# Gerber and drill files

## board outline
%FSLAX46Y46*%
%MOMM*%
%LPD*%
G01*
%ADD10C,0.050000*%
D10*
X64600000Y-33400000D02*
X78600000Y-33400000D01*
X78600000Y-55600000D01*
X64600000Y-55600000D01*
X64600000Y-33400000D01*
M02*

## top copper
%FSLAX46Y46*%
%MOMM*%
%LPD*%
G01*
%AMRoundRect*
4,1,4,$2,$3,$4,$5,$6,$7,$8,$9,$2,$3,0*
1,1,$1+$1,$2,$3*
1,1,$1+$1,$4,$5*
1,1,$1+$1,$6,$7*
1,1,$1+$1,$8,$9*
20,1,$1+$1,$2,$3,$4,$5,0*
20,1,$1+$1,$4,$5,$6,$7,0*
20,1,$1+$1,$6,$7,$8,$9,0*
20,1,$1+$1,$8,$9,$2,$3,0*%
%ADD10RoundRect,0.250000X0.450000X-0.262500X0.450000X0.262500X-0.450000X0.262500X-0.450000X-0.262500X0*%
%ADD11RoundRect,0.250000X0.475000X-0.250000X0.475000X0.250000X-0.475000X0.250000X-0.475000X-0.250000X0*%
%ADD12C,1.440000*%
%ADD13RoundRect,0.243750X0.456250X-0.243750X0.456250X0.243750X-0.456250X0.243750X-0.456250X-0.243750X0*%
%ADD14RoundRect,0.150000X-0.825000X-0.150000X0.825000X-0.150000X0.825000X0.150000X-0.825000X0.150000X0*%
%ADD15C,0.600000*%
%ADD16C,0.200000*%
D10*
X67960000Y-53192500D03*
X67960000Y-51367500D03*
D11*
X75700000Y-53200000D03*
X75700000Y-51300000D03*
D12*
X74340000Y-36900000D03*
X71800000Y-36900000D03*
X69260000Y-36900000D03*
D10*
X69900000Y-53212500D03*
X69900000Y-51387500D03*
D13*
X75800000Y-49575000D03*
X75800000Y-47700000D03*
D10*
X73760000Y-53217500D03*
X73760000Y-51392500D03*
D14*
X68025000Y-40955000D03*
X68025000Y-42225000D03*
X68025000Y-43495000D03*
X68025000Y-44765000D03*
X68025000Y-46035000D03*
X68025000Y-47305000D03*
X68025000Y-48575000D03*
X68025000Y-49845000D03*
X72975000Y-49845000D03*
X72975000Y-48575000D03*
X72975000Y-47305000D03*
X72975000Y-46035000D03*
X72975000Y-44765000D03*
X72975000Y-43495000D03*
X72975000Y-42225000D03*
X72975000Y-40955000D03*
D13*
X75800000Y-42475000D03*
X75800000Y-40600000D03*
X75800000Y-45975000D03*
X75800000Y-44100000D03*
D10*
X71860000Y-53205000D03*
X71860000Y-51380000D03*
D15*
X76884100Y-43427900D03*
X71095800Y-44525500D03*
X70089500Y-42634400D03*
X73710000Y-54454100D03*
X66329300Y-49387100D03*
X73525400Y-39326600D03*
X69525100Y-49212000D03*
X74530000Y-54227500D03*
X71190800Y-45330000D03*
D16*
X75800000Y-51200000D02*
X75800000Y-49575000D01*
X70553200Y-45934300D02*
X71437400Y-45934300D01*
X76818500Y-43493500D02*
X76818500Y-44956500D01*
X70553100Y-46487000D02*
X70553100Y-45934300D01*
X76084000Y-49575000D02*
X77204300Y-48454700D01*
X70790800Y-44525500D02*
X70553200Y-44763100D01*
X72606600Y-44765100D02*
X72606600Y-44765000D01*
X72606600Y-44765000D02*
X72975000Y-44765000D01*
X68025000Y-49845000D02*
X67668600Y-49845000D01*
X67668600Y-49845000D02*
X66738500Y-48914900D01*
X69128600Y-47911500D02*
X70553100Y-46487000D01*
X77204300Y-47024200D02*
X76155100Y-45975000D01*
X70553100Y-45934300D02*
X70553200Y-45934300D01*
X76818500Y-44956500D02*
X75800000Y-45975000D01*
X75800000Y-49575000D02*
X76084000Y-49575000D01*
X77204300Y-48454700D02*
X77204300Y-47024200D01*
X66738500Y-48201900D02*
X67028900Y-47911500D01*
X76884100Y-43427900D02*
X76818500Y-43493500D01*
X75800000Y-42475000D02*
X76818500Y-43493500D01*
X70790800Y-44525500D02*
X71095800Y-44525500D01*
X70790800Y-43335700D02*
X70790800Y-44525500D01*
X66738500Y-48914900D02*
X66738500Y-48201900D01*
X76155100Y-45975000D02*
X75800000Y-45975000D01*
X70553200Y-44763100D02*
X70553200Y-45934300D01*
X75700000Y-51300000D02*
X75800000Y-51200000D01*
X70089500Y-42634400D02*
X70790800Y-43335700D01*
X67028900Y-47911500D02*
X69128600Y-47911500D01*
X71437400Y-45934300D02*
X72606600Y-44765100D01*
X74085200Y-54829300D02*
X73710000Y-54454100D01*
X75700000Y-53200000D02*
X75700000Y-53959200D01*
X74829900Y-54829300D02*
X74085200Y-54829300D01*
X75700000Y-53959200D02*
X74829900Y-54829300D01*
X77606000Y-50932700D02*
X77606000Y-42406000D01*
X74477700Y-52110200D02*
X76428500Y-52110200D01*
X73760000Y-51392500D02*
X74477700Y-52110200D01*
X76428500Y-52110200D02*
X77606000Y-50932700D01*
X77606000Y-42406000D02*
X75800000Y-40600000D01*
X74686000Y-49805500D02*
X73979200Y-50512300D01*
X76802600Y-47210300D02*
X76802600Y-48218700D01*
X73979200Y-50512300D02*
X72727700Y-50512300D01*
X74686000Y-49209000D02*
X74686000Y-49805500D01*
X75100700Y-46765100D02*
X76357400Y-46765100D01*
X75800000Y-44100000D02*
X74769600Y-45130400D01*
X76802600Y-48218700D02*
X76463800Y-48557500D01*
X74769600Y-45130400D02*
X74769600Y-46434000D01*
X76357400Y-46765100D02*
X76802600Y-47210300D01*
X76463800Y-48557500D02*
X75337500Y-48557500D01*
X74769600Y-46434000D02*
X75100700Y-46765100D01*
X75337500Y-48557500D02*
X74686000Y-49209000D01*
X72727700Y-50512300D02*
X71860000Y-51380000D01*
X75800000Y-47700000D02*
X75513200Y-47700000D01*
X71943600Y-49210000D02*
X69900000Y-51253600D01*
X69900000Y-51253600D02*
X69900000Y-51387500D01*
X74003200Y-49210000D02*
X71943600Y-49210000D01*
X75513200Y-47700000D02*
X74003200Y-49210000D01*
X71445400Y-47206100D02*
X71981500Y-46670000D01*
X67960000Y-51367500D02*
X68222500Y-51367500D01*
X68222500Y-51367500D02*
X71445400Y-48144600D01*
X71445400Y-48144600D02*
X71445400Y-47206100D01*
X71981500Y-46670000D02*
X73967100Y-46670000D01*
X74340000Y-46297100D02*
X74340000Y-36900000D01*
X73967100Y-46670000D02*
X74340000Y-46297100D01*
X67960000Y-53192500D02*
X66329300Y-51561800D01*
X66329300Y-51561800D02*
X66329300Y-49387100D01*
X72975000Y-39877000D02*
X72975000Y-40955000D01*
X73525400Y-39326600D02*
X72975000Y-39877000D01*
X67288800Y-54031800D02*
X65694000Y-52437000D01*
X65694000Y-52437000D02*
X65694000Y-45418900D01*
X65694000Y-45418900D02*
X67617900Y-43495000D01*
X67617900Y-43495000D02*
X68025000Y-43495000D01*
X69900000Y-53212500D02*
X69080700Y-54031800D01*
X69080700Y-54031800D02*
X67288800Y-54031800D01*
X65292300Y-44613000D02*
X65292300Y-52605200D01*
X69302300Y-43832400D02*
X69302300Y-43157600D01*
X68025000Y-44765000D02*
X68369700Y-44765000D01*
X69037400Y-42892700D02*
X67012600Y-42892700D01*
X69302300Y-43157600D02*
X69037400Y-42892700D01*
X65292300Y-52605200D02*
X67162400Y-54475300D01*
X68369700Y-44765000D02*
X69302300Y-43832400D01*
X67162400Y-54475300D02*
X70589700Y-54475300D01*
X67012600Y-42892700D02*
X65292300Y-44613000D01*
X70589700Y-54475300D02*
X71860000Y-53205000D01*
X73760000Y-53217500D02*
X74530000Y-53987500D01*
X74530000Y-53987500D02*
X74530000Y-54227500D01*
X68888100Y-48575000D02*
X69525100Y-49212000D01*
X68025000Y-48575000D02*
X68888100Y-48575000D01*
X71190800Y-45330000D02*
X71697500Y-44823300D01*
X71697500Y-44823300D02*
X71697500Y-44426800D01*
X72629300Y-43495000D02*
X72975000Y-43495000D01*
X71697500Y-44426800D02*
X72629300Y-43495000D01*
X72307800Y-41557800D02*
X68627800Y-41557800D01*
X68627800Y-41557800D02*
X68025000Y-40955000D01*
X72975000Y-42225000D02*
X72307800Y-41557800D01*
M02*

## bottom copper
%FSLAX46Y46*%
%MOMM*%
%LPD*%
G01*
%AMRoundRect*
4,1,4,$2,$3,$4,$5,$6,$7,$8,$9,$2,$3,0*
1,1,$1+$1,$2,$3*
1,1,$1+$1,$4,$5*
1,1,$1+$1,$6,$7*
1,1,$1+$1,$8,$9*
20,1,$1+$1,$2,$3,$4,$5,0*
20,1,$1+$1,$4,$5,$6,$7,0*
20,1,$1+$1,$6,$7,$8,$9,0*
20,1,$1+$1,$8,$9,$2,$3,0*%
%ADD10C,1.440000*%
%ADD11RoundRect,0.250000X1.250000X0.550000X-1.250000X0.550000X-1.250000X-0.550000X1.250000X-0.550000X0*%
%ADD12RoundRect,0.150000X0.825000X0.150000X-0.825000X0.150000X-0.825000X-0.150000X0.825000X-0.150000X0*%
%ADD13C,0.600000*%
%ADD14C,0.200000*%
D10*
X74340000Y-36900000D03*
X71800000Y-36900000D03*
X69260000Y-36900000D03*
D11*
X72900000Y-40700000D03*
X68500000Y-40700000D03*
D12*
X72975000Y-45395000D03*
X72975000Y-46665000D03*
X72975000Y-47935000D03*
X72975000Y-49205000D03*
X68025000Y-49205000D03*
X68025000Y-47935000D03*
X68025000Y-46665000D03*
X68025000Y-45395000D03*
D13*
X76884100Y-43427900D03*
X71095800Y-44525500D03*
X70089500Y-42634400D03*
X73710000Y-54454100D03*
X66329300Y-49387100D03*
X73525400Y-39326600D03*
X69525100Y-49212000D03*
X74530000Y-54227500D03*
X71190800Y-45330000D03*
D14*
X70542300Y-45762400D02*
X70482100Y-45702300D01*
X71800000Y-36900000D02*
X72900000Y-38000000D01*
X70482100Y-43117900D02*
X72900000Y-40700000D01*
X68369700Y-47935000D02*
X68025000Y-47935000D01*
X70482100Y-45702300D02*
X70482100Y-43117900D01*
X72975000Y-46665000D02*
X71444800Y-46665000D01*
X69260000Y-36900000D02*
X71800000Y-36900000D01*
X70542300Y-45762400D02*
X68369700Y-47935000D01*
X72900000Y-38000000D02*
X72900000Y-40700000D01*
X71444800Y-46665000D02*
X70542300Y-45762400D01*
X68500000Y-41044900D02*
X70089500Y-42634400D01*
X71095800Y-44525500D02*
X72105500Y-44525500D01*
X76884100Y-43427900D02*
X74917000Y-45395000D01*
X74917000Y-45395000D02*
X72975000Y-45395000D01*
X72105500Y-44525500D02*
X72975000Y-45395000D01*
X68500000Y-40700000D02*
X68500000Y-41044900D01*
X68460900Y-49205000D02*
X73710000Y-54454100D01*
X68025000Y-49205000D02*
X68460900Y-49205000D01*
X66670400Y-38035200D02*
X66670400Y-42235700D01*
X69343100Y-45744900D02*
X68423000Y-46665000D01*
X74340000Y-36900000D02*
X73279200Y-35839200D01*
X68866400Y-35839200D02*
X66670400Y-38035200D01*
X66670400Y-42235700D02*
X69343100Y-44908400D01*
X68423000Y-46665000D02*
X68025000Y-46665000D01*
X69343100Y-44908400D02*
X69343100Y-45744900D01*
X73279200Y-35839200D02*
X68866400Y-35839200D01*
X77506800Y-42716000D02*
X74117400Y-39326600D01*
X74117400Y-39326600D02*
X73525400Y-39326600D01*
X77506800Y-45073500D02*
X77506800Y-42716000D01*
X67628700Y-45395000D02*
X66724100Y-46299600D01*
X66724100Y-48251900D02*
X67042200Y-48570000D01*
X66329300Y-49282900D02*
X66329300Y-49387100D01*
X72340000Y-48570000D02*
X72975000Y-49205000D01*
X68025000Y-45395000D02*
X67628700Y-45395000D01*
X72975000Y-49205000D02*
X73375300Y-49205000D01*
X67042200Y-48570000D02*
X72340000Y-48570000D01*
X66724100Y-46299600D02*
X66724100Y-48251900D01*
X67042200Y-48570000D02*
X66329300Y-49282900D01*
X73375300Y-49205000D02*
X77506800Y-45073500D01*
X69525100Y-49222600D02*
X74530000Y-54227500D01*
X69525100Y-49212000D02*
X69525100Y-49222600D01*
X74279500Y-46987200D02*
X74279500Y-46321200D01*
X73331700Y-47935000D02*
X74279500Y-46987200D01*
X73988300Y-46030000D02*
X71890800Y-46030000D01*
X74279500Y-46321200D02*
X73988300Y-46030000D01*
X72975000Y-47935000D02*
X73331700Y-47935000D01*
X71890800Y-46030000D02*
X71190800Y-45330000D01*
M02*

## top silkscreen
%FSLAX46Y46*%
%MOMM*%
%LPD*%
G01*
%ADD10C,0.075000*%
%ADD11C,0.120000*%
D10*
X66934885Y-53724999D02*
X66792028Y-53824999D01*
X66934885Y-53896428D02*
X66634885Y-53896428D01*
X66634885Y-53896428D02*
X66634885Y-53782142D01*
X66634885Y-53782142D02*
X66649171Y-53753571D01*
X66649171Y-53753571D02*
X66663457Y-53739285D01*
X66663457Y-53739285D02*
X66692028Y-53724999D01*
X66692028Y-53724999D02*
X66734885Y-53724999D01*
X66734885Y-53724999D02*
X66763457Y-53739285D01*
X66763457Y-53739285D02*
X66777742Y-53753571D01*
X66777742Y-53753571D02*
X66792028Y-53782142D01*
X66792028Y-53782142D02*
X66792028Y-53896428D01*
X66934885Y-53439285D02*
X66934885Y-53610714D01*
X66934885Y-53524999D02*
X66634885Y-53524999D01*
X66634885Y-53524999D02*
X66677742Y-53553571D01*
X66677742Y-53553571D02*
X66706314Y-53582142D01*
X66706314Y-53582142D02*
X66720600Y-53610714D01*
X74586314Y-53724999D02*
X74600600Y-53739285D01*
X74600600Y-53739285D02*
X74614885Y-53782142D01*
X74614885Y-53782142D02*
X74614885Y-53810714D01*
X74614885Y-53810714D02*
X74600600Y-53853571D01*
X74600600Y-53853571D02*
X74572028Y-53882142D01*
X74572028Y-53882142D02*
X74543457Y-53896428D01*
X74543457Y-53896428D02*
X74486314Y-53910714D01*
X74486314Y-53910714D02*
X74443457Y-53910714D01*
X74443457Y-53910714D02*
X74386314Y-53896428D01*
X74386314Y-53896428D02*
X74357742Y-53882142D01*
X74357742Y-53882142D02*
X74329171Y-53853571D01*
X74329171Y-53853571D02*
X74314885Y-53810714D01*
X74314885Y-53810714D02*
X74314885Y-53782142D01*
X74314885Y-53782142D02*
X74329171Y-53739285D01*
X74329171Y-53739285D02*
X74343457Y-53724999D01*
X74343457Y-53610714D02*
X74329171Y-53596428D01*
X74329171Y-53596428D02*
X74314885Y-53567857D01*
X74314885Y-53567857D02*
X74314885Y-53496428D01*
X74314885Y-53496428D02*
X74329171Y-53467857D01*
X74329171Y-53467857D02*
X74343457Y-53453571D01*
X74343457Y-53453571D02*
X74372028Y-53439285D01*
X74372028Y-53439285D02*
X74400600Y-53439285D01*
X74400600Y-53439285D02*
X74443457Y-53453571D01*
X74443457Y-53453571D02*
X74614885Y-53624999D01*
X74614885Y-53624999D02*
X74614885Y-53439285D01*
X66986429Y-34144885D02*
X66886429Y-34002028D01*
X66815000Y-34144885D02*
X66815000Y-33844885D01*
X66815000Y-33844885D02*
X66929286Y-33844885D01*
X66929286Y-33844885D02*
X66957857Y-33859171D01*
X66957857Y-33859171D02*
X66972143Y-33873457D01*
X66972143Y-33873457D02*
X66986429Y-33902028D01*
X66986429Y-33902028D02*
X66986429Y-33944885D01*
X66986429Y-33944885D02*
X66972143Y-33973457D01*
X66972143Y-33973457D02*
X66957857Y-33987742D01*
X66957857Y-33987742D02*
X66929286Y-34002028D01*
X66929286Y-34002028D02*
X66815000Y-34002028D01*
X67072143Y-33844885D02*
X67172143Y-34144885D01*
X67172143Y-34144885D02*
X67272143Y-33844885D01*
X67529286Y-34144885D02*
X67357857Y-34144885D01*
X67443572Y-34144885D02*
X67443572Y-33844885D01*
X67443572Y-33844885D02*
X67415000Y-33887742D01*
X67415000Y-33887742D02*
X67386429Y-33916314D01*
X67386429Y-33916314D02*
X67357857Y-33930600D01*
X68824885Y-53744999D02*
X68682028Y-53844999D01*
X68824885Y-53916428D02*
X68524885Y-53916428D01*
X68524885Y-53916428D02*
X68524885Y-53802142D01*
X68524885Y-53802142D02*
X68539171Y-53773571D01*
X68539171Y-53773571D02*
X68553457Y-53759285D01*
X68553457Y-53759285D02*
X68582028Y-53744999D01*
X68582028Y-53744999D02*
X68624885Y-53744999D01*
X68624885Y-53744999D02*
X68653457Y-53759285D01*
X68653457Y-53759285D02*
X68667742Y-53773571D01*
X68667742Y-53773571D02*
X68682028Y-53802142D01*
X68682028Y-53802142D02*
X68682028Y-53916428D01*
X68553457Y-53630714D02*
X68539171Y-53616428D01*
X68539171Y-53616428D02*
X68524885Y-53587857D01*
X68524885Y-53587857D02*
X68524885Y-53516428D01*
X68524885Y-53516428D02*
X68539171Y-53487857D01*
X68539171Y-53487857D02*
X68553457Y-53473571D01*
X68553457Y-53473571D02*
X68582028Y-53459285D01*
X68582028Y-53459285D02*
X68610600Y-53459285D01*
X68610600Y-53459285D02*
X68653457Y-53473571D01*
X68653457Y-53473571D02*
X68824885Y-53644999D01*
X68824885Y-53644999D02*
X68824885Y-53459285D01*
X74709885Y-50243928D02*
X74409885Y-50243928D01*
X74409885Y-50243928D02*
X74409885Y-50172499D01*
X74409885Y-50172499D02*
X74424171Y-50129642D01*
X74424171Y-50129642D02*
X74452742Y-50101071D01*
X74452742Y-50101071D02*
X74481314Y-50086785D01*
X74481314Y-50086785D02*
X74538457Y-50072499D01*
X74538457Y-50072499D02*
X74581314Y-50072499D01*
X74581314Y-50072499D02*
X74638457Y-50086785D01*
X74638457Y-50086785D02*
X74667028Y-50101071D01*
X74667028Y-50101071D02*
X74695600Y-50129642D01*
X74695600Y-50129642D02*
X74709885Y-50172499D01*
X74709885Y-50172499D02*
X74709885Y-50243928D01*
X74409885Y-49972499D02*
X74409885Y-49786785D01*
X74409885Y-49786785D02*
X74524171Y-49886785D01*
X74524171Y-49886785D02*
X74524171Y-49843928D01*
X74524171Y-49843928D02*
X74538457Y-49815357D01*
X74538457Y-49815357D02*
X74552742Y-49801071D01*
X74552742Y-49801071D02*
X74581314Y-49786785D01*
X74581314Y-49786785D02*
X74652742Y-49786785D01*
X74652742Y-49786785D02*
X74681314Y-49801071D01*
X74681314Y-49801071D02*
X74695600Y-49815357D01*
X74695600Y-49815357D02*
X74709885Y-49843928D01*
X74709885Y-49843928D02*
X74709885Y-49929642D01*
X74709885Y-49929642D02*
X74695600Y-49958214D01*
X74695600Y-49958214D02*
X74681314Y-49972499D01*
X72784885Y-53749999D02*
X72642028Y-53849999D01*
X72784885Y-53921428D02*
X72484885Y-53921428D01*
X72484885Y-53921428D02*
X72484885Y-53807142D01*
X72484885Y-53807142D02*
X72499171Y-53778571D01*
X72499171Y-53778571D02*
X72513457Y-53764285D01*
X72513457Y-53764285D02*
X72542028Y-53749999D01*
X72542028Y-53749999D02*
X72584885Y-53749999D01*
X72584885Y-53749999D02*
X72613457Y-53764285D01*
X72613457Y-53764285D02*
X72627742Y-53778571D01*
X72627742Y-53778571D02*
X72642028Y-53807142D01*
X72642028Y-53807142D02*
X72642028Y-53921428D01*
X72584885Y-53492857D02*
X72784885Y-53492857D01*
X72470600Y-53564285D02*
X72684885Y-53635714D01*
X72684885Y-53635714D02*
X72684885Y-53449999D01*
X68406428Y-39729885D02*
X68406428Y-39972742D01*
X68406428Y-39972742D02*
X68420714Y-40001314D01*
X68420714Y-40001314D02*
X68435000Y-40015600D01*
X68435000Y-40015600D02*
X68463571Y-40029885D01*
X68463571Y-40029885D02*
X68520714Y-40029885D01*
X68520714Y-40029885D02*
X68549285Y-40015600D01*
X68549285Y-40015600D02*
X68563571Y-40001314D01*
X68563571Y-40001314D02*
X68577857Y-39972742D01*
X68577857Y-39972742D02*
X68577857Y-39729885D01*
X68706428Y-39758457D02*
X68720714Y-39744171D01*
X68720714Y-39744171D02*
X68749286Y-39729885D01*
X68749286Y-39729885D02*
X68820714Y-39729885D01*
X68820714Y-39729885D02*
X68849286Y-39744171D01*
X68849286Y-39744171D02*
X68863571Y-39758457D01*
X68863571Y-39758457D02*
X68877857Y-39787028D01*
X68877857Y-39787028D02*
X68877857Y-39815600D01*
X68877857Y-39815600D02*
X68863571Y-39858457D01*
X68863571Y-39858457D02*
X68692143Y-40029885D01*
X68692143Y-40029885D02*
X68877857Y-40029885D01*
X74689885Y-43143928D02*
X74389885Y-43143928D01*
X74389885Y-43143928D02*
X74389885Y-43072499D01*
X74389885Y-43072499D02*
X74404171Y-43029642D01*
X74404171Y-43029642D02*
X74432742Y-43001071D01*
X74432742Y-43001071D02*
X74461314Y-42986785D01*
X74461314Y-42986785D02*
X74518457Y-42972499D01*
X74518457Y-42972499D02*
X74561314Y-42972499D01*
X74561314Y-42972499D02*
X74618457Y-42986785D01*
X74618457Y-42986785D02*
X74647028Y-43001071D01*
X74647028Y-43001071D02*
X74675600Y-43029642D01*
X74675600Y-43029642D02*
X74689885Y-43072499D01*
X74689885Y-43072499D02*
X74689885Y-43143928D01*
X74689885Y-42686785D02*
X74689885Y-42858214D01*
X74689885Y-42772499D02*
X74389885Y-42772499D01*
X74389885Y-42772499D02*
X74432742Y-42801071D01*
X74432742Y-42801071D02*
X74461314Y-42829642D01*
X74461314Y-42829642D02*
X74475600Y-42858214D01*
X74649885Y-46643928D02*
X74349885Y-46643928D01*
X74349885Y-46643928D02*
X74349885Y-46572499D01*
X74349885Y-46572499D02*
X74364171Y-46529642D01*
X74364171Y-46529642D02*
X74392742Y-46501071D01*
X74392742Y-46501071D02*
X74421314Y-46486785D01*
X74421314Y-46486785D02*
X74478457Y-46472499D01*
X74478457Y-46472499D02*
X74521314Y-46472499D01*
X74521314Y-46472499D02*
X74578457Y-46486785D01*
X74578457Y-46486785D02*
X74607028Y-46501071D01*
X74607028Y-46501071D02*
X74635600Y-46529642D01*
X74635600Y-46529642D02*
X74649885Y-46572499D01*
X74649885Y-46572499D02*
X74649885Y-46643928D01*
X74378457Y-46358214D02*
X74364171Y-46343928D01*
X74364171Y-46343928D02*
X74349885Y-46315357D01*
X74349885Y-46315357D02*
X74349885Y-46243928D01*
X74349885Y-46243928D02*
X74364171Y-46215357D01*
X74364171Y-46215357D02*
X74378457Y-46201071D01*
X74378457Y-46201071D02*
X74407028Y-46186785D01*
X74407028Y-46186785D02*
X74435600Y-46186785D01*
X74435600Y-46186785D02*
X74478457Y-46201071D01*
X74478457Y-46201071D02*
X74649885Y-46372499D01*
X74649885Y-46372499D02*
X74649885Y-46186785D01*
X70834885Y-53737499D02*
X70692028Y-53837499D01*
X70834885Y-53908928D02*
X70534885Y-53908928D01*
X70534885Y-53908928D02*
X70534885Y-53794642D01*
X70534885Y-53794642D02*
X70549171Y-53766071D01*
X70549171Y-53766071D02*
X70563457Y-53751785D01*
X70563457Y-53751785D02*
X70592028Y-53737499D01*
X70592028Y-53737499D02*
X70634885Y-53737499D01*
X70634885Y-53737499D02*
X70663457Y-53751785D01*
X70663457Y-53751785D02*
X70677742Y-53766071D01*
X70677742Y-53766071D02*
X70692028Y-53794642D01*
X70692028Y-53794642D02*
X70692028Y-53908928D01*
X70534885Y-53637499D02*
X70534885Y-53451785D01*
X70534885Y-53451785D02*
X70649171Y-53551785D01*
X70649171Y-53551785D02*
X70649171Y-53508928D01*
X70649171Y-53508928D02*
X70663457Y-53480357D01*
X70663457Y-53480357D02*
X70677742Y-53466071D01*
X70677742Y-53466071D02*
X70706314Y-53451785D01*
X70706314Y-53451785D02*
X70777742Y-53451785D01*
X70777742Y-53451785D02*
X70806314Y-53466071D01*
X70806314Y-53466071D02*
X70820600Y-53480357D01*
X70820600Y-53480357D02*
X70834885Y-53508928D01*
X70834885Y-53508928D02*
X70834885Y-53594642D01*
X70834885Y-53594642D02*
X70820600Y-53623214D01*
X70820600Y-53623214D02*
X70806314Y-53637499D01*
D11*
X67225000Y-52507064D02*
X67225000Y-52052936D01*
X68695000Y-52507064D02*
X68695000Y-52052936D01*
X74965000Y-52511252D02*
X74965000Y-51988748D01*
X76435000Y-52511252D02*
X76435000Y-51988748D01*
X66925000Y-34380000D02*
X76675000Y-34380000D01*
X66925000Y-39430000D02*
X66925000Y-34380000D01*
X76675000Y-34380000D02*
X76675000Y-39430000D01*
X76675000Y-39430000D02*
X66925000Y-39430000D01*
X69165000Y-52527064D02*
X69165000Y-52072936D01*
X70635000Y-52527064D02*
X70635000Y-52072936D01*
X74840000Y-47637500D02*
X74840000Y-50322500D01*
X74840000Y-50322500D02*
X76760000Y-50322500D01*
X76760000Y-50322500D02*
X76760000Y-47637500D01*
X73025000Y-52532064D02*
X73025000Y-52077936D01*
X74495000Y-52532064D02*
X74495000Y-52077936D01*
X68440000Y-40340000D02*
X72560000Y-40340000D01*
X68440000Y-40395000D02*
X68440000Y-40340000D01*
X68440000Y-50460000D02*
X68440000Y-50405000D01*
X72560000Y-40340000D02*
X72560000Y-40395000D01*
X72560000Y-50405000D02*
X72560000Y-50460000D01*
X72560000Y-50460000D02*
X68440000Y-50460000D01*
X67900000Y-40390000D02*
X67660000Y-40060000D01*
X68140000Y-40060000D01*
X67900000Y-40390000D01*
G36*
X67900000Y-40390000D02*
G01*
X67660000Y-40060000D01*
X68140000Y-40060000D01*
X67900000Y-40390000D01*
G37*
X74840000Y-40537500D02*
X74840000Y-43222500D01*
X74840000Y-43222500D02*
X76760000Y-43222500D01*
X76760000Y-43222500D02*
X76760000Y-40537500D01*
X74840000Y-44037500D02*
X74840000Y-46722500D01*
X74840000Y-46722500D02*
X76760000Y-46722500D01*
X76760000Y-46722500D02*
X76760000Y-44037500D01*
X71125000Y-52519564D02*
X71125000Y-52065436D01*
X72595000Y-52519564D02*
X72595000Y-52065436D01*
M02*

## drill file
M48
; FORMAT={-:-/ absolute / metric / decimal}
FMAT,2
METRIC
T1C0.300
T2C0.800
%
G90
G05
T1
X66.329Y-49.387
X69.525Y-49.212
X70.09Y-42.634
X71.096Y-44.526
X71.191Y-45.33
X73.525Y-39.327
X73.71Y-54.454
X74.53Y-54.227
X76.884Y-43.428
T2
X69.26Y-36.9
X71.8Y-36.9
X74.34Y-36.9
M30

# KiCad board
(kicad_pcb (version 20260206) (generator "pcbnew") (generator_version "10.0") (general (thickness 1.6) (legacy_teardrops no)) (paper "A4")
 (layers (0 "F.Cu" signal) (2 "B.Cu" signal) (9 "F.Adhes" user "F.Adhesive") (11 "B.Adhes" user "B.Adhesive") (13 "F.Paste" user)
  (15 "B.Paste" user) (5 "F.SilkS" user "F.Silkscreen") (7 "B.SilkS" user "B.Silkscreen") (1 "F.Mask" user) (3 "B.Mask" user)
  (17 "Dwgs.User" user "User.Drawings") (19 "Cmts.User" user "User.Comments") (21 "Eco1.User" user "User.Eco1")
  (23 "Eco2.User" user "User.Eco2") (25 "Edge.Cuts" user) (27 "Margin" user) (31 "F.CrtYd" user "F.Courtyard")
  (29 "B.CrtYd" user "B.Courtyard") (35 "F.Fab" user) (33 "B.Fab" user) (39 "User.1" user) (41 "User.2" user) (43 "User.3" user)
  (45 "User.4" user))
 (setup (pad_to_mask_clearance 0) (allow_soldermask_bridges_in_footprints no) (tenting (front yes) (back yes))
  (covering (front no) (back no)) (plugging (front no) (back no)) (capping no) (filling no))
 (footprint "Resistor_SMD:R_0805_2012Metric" (layer "F.Cu") (at 67.96 52.28 90)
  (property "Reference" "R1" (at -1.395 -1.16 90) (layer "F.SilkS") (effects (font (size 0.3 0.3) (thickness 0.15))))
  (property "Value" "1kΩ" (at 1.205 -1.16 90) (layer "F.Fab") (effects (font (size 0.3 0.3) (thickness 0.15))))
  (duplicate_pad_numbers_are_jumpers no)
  (fp_line (start -0.227064 -0.735) (end 0.227064 -0.735) (stroke (width 0.12) (type solid)) (layer "F.SilkS"))
  (fp_line (start -0.227064 0.735) (end 0.227064 0.735) (stroke (width 0.12) (type solid)) (layer "F.SilkS"))
  (pad "1" smd roundrect (at -0.9125 0 90) (size 1.025 1.4) (layers "F.Cu" "F.Mask" "F.Paste") (roundrect_rratio 0.243902) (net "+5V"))
  (pad "2" smd roundrect (at 0.9125 0 90) (size 1.025 1.4) (layers "F.Cu" "F.Mask" "F.Paste") (roundrect_rratio 0.243902) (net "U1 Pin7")))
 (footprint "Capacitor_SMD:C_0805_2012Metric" (layer "F.Cu") (at 75.7 52.25 90)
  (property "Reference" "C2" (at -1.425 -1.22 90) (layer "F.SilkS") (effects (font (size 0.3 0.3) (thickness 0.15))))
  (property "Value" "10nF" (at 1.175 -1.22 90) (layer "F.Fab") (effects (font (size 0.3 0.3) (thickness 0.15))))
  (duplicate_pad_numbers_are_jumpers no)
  (fp_line (start -0.261252 -0.735) (end 0.261252 -0.735) (stroke (width 0.12) (type solid)) (layer "F.SilkS"))
  (fp_line (start -0.261252 0.735) (end 0.261252 0.735) (stroke (width 0.12) (type solid)) (layer "F.SilkS"))
  (pad "1" smd roundrect (at -0.95 0 90) (size 1 1.45) (layers "F.Cu" "F.Mask" "F.Paste") (roundrect_rratio 0.25) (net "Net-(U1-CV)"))
  (pad "2" smd roundrect (at 0.95 0 90) (size 1 1.45) (layers "F.Cu" "F.Mask" "F.Paste") (roundrect_rratio 0.25) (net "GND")))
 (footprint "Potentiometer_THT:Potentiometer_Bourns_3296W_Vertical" (layer "F.Cu") (at 74.34 36.9)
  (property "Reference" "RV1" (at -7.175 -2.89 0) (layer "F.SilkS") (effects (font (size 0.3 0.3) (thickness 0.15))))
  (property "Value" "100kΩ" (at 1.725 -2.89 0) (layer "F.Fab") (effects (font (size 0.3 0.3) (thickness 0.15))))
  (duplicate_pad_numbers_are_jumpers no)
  (fp_line (start -7.415 -2.52) (end 2.335 -2.52) (stroke (width 0.12) (type solid)) (layer "F.SilkS"))
  (fp_line (start -7.415 2.53) (end -7.415 -2.52) (stroke (width 0.12) (type solid)) (layer "F.SilkS"))
  (fp_line (start 2.335 -2.52) (end 2.335 2.53) (stroke (width 0.12) (type solid)) (layer "F.SilkS"))
  (fp_line (start 2.335 2.53) (end -7.415 2.53) (stroke (width 0.12) (type solid)) (layer "F.SilkS"))
  (pad "1" thru_hole circle (at 0 0) (size 1.44 1.44) (drill 0.8) (layers "*.Cu" "*.Mask") (remove_unused_layers no) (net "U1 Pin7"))
  (pad "2" thru_hole circle (at -2.54 0) (size 1.44 1.44) (drill 0.8) (layers "*.Cu" "*.Mask") (remove_unused_layers no) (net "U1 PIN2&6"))
  (pad "3" thru_hole circle (at -5.08 0) (size 1.44 1.44) (drill 0.8) (layers "*.Cu" "*.Mask") (remove_unused_layers no) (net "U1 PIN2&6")))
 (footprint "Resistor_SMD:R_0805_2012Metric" (layer "F.Cu") (at 69.9 52.3 90)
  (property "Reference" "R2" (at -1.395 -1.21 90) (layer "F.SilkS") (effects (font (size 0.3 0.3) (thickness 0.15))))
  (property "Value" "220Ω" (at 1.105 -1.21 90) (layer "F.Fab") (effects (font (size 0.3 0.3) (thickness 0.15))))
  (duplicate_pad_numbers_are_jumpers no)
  (fp_line (start -0.227064 -0.735) (end 0.227064 -0.735) (stroke (width 0.12) (type solid)) (layer "F.SilkS"))
  (fp_line (start -0.227064 0.735) (end 0.227064 0.735) (stroke (width 0.12) (type solid)) (layer "F.SilkS"))
  (pad "1" smd roundrect (at -0.9125 0 90) (size 1.025 1.4) (layers "F.Cu" "F.Mask" "F.Paste") (roundrect_rratio 0.243902) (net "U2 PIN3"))
  (pad "2" smd roundrect (at 0.9125 0 90) (size 1.025 1.4) (layers "F.Cu" "F.Mask" "F.Paste") (roundrect_rratio 0.243902) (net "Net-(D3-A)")))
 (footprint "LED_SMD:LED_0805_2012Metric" (layer "F.Cu") (at 75.8 48.6375 90)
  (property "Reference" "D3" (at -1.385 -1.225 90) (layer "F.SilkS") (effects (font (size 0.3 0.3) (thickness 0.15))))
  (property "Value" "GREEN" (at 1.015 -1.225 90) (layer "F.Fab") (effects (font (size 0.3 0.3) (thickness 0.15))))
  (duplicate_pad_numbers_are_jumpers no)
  (fp_line (start 1 -0.96) (end -1.685 -0.96) (stroke (width 0.12) (type solid)) (layer "F.SilkS"))
  (fp_line (start -1.685 -0.96) (end -1.685 0.96) (stroke (width 0.12) (type solid)) (layer "F.SilkS"))
  (fp_line (start -1.685 0.96) (end 1 0.96) (stroke (width 0.12) (type solid)) (layer "F.SilkS"))
  (pad "1" smd roundrect (at -0.9375 0 90) (size 0.975 1.4) (layers "F.Cu" "F.Mask" "F.Paste") (roundrect_rratio 0.25) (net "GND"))
  (pad "2" smd roundrect (at 0.9375 0 90) (size 0.975 1.4) (layers "F.Cu" "F.Mask" "F.Paste") (roundrect_rratio 0.25) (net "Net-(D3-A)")))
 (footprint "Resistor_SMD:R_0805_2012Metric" (layer "F.Cu") (at 73.76 52.305 90)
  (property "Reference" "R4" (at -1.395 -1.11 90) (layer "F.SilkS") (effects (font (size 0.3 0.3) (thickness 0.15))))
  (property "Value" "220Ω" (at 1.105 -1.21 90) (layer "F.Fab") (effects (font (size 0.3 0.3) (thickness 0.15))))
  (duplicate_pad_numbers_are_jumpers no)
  (fp_line (start -0.227064 -0.735) (end 0.227064 -0.735) (stroke (width 0.12) (type solid)) (layer "F.SilkS"))
  (fp_line (start -0.227064 0.735) (end 0.227064 0.735) (stroke (width 0.12) (type solid)) (layer "F.SilkS"))
  (pad "1" smd roundrect (at -0.9125 0 90) (size 1.025 1.4) (layers "F.Cu" "F.Mask" "F.Paste") (roundrect_rratio 0.243902) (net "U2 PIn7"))
  (pad "2" smd roundrect (at 0.9125 0 90) (size 1.025 1.4) (layers "F.Cu" "F.Mask" "F.Paste") (roundrect_rratio 0.243902) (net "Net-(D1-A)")))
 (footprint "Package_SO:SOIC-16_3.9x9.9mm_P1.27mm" (layer "F.Cu") (at 70.5 45.4)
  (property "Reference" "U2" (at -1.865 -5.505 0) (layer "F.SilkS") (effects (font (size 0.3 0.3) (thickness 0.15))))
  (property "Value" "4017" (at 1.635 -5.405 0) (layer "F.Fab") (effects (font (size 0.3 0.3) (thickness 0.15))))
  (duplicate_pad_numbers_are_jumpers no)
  (fp_line (start -2.06 -5.06) (end 2.06 -5.06) (stroke (width 0.12) (type solid)) (layer "F.SilkS"))
  (fp_line (start -2.06 -5.005) (end -2.06 -5.06) (stroke (width 0.12) (type solid)) (layer "F.SilkS"))
  (fp_line (start -2.06 5.06) (end -2.06 5.005) (stroke (width 0.12) (type solid)) (layer "F.SilkS"))
  (fp_line (start 2.06 -5.06) (end 2.06 -5.005) (stroke (width 0.12) (type solid)) (layer "F.SilkS"))
  (fp_line (start 2.06 5.005) (end 2.06 5.06) (stroke (width 0.12) (type solid)) (layer "F.SilkS"))
  (fp_line (start 2.06 5.06) (end -2.06 5.06) (stroke (width 0.12) (type solid)) (layer "F.SilkS"))
  (fp_poly (pts (xy -2.6 -5.01) (xy -2.84 -5.34) (xy -2.36 -5.34)) (stroke (width 0.12) (type solid)) (fill yes) (layer "F.SilkS"))
  (pad "1" smd roundrect (at -2.475 -4.445) (size 1.95 0.6) (layers "F.Cu" "F.Mask" "F.Paste") (roundrect_rratio 0.25) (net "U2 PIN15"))
  (pad "2" smd roundrect (at -2.475 -3.175) (size 1.95 0.6) (layers "F.Cu" "F.Mask" "F.Paste") (roundrect_rratio 0.25)
   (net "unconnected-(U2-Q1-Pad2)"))
  (pad "3" smd roundrect (at -2.475 -1.905) (size 1.95 0.6) (layers "F.Cu" "F.Mask" "F.Paste") (roundrect_rratio 0.25) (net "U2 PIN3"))
  (pad "4" smd roundrect (at -2.475 -0.635) (size 1.95 0.6) (layers "F.Cu" "F.Mask" "F.Paste") (roundrect_rratio 0.25) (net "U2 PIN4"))
  (pad "5" smd roundrect (at -2.475 0.635) (size 1.95 0.6) (layers "F.Cu" "F.Mask" "F.Paste") (roundrect_rratio 0.25)
   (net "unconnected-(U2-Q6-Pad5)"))
  (pad "6" smd roundrect (at -2.475 1.905) (size 1.95 0.6) (layers "F.Cu" "F.Mask" "F.Paste") (roundrect_rratio 0.25)
   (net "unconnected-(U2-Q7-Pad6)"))
  (pad "7" smd roundrect (at -2.475 3.175) (size 1.95 0.6) (layers "F.Cu" "F.Mask" "F.Paste") (roundrect_rratio 0.25) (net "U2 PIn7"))
  (pad "8" smd roundrect (at -2.475 4.445) (size 1.95 0.6) (layers "F.Cu" "F.Mask" "F.Paste") (roundrect_rratio 0.25) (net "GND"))
  (pad "9" smd roundrect (at 2.475 4.445) (size 1.95 0.6) (layers "F.Cu" "F.Mask" "F.Paste") (roundrect_rratio 0.25)
   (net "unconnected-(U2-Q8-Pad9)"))
  (pad "10" smd roundrect (at 2.475 3.175) (size 1.95 0.6) (layers "F.Cu" "F.Mask" "F.Paste") (roundrect_rratio 0.25)
   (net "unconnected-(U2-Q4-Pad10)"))
  (pad "11" smd roundrect (at 2.475 1.905) (size 1.95 0.6) (layers "F.Cu" "F.Mask" "F.Paste") (roundrect_rratio 0.25)
   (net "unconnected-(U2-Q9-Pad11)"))
  (pad "12" smd roundrect (at 2.475 0.635) (size 1.95 0.6) (layers "F.Cu" "F.Mask" "F.Paste") (roundrect_rratio 0.25)
   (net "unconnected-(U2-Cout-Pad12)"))
  (pad "13" smd roundrect (at 2.475 -0.635) (size 1.95 0.6) (layers "F.Cu" "F.Mask" "F.Paste") (roundrect_rratio 0.25) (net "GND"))
  (pad "14" smd roundrect (at 2.475 -1.905) (size 1.95 0.6) (layers "F.Cu" "F.Mask" "F.Paste") (roundrect_rratio 0.25) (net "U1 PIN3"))
  (pad "15" smd roundrect (at 2.475 -3.175) (size 1.95 0.6) (layers "F.Cu" "F.Mask" "F.Paste") (roundrect_rratio 0.25) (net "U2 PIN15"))
  (pad "16" smd roundrect (at 2.475 -4.445) (size 1.95 0.6) (layers "F.Cu" "F.Mask" "F.Paste") (roundrect_rratio 0.25) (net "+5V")))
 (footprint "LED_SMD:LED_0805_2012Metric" (layer "F.Cu") (at 75.8 41.5375 90)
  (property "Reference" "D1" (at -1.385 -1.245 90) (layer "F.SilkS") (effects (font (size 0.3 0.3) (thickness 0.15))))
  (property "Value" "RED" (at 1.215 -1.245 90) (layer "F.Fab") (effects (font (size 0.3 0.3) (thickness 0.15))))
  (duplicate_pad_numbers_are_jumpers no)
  (fp_line (start 1 -0.96) (end -1.685 -0.96) (stroke (width 0.12) (type solid)) (layer "F.SilkS"))
  (fp_line (start -1.685 -0.96) (end -1.685 0.96) (stroke (width 0.12) (type solid)) (layer "F.SilkS"))
  (fp_line (start -1.685 0.96) (end 1 0.96) (stroke (width 0.12) (type solid)) (layer "F.SilkS"))
  (pad "1" smd roundrect (at -0.9375 0 90) (size 0.975 1.4) (layers "F.Cu" "F.Mask" "F.Paste") (roundrect_rratio 0.25) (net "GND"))
  (pad "2" smd roundrect (at 0.9375 0 90) (size 0.975 1.4) (layers "F.Cu" "F.Mask" "F.Paste") (roundrect_rratio 0.25) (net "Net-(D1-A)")))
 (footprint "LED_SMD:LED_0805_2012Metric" (layer "F.Cu") (at 75.8 45.0375 90)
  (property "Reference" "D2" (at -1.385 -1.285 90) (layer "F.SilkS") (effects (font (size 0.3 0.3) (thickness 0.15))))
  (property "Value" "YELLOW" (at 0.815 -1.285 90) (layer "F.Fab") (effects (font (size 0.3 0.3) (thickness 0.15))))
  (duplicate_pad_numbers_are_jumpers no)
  (fp_line (start 1 -0.96) (end -1.685 -0.96) (stroke (width 0.12) (type solid)) (layer "F.SilkS"))
  (fp_line (start -1.685 -0.96) (end -1.685 0.96) (stroke (width 0.12) (type solid)) (layer "F.SilkS"))
  (fp_line (start -1.685 0.96) (end 1 0.96) (stroke (width 0.12) (type solid)) (layer "F.SilkS"))
  (pad "1" smd roundrect (at -0.9375 0 90) (size 0.975 1.4) (layers "F.Cu" "F.Mask" "F.Paste") (roundrect_rratio 0.25) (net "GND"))
  (pad "2" smd roundrect (at 0.9375 0 90) (size 0.975 1.4) (layers "F.Cu" "F.Mask" "F.Paste") (roundrect_rratio 0.25) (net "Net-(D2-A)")))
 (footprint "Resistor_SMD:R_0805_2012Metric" (layer "F.Cu") (at 71.86 52.2925 90)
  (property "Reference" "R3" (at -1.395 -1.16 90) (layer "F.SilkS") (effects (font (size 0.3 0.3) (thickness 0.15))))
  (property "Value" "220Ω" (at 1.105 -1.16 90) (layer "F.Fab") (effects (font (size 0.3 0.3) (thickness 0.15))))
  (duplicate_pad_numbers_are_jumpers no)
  (fp_line (start -0.227064 -0.735) (end 0.227064 -0.735) (stroke (width 0.12) (type solid)) (layer "F.SilkS"))
  (fp_line (start -0.227064 0.735) (end 0.227064 0.735) (stroke (width 0.12) (type solid)) (layer "F.SilkS"))
  (pad "1" smd roundrect (at -0.9125 0 90) (size 1.025 1.4) (layers "F.Cu" "F.Mask" "F.Paste") (roundrect_rratio 0.243902) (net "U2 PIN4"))
  (pad "2" smd roundrect (at 0.9125 0 90) (size 1.025 1.4) (layers "F.Cu" "F.Mask" "F.Paste") (roundrect_rratio 0.243902) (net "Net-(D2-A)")))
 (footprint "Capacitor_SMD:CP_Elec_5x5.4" (layer "B.Cu") (at 70.7 40.7 180)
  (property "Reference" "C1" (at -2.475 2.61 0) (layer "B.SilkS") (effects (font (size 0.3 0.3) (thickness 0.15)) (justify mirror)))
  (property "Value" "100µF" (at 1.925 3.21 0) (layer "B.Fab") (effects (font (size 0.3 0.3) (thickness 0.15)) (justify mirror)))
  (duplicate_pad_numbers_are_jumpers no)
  (pad "1" smd roundrect (at -2.2 0 180) (size 3 1.6) (layers "B.Cu" "B.Mask" "B.Paste") (roundrect_rratio 0.15625) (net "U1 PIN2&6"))
  (pad "2" smd roundrect (at 2.2 0 180) (size 3 1.6) (layers "B.Cu" "B.Mask" "B.Paste") (roundrect_rratio 0.15625) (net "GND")))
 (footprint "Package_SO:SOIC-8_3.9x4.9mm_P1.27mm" (layer "B.Cu") (at 70.5 47.3 180)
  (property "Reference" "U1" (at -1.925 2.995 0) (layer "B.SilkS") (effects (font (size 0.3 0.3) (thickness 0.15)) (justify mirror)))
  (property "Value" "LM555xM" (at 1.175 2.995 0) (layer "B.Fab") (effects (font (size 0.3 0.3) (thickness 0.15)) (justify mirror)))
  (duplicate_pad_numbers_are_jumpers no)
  (pad "1" smd roundrect (at -2.475 1.905 180) (size 1.95 0.6) (layers "B.Cu" "B.Mask" "B.Paste") (roundrect_rratio 0.25) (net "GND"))
  (pad "2" smd roundrect (at -2.475 0.635 180) (size 1.95 0.6) (layers "B.Cu" "B.Mask" "B.Paste") (roundrect_rratio 0.25) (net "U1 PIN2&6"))
  (pad "3" smd roundrect (at -2.475 -0.635 180) (size 1.95 0.6) (layers "B.Cu" "B.Mask" "B.Paste") (roundrect_rratio 0.25) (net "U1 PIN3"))
  (pad "4" smd roundrect (at -2.475 -1.905 180) (size 1.95 0.6) (layers "B.Cu" "B.Mask" "B.Paste") (roundrect_rratio 0.25) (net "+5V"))
  (pad "5" smd roundrect (at 2.475 -1.905 180) (size 1.95 0.6) (layers "B.Cu" "B.Mask" "B.Paste") (roundrect_rratio 0.25)
   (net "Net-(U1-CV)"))
  (pad "6" smd roundrect (at 2.475 -0.635 180) (size 1.95 0.6) (layers "B.Cu" "B.Mask" "B.Paste") (roundrect_rratio 0.25) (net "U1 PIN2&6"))
  (pad "7" smd roundrect (at 2.475 0.635 180) (size 1.95 0.6) (layers "B.Cu" "B.Mask" "B.Paste") (roundrect_rratio 0.25) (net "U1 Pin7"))
  (pad "8" smd roundrect (at 2.475 1.905 180) (size 1.95 0.6) (layers "B.Cu" "B.Mask" "B.Paste") (roundrect_rratio 0.25) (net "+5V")))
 (gr_rect (start 64.6 33.4) (end 78.6 55.6) (stroke (width 0.05) (type default)) (fill no) (layer "Edge.Cuts"))
 (segment (start 70.5423 45.7624) (end 70.4821 45.7023) (width 0.2) (layer "B.Cu") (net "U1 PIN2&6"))
 (segment (start 71.8 36.9) (end 72.9 38) (width 0.2) (layer "B.Cu") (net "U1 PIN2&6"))
 (segment (start 70.4821 43.1179) (end 72.9 40.7) (width 0.2) (layer "B.Cu") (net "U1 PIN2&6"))
 (segment (start 68.3697 47.935) (end 68.025 47.935) (width 0.2) (layer "B.Cu") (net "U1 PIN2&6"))
 (segment (start 70.4821 45.7023) (end 70.4821 43.1179) (width 0.2) (layer "B.Cu") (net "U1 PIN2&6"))
 (segment (start 72.975 46.665) (end 71.4448 46.665) (width 0.2) (layer "B.Cu") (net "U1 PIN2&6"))
 (segment (start 69.26 36.9) (end 71.8 36.9) (width 0.2) (layer "B.Cu") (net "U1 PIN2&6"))
 (segment (start 70.5423 45.7624) (end 68.3697 47.935) (width 0.2) (layer "B.Cu") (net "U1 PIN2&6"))
 (segment (start 72.9 38) (end 72.9 40.7) (width 0.2) (layer "B.Cu") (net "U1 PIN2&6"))
 (segment (start 71.4448 46.665) (end 70.5423 45.7624) (width 0.2) (layer "B.Cu") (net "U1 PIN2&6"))
 (segment (start 75.8 51.2) (end 75.8 49.575) (width 0.2) (layer "F.Cu") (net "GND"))
 (segment (start 70.5532 45.9343) (end 71.4374 45.9343) (width 0.2) (layer "F.Cu") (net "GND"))
 (segment (start 76.8185 43.4935) (end 76.8185 44.9565) (width 0.2) (layer "F.Cu") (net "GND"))
 (segment (start 70.5531 46.487) (end 70.5531 45.9343) (width 0.2) (layer "F.Cu") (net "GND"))
 (segment (start 76.084 49.575) (end 77.2043 48.4547) (width 0.2) (layer "F.Cu") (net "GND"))
 (segment (start 70.7908 44.5255) (end 70.5532 44.7631) (width 0.2) (layer "F.Cu") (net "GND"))
 (segment (start 72.6066 44.7651) (end 72.6066 44.765) (width 0.2) (layer "F.Cu") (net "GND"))
 (segment (start 72.6066 44.765) (end 72.975 44.765) (width 0.2) (layer "F.Cu") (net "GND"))
 (segment (start 68.025 49.845) (end 67.6686 49.845) (width 0.2) (layer "F.Cu") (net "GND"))
 (segment (start 67.6686 49.845) (end 66.7385 48.9149) (width 0.2) (layer "F.Cu") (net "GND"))
 (segment (start 69.1286 47.9115) (end 70.5531 46.487) (width 0.2) (layer "F.Cu") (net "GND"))
 (segment (start 77.2043 47.0242) (end 76.1551 45.975) (width 0.2) (layer "F.Cu") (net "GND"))
 (segment (start 70.5531 45.9343) (end 70.5532 45.9343) (width 0.2) (layer "F.Cu") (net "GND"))
 (segment (start 76.8185 44.9565) (end 75.8 45.975) (width 0.2) (layer "F.Cu") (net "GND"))
 (segment (start 75.8 49.575) (end 76.084 49.575) (width 0.2) (layer "F.Cu") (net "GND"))
 (segment (start 77.2043 48.4547) (end 77.2043 47.0242) (width 0.2) (layer "F.Cu") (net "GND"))
 (segment (start 66.7385 48.2019) (end 67.0289 47.9115) (width 0.2) (layer "F.Cu") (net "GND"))
 (segment (start 76.8841 43.4279) (end 76.8185 43.4935) (width 0.2) (layer "F.Cu") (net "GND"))
 (segment (start 75.8 42.475) (end 76.8185 43.4935) (width 0.2) (layer "F.Cu") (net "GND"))
 (segment (start 70.7908 44.5255) (end 71.0958 44.5255) (width 0.2) (layer "F.Cu") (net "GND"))
 (segment (start 70.7908 43.3357) (end 70.7908 44.5255) (width 0.2) (layer "F.Cu") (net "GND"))
 (segment (start 66.7385 48.9149) (end 66.7385 48.2019) (width 0.2) (layer "F.Cu") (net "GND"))
 (segment (start 76.1551 45.975) (end 75.8 45.975) (width 0.2) (layer "F.Cu") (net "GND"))
 (segment (start 70.5532 44.7631) (end 70.5532 45.9343) (width 0.2) (layer "F.Cu") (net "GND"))
 (segment (start 75.7 51.3) (end 75.8 51.2) (width 0.2) (layer "F.Cu") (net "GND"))
 (segment (start 70.0895 42.6344) (end 70.7908 43.3357) (width 0.2) (layer "F.Cu") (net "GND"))
 (segment (start 67.0289 47.9115) (end 69.1286 47.9115) (width 0.2) (layer "F.Cu") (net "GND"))
 (segment (start 71.4374 45.9343) (end 72.6066 44.7651) (width 0.2) (layer "F.Cu") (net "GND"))
 (via (at 76.8841 43.4279) (size 0.6) (drill 0.3) (layers "F.Cu" "B.Cu") (capping no) (covering (front no) (back no))
  (plugging (front no) (back no)) (filling no) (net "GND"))
 (via (at 71.0958 44.5255) (size 0.6) (drill 0.3) (layers "F.Cu" "B.Cu") (capping no) (covering (front no) (back no))
  (plugging (front no) (back no)) (filling no) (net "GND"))
 (via (at 70.0895 42.6344) (size 0.6) (drill 0.3) (layers "F.Cu" "B.Cu") (capping no) (covering (front no) (back no))
  (plugging (front no) (back no)) (filling no) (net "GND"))
 (segment (start 68.5 41.0449) (end 70.0895 42.6344) (width 0.2) (layer "B.Cu") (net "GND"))
 (segment (start 71.0958 44.5255) (end 72.1055 44.5255) (width 0.2) (layer "B.Cu") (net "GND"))
 (segment (start 76.8841 43.4279) (end 74.917 45.395) (width 0.2) (layer "B.Cu") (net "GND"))
 (segment (start 74.917 45.395) (end 72.975 45.395) (width 0.2) (layer "B.Cu") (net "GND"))
 (segment (start 72.1055 44.5255) (end 72.975 45.395) (width 0.2) (layer "B.Cu") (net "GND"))
 (segment (start 68.5 40.7) (end 68.5 41.0449) (width 0.2) (layer "B.Cu") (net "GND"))
 (segment (start 74.0852 54.8293) (end 73.71 54.4541) (width 0.2) (layer "F.Cu") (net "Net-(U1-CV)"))
 (segment (start 75.7 53.2) (end 75.7 53.9592) (width 0.2) (layer "F.Cu") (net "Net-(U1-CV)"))
 (segment (start 74.8299 54.8293) (end 74.0852 54.8293) (width 0.2) (layer "F.Cu") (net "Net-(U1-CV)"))
 (segment (start 75.7 53.9592) (end 74.8299 54.8293) (width 0.2) (layer "F.Cu") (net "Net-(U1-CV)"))
 (via (at 73.71 54.4541) (size 0.6) (drill 0.3) (layers "F.Cu" "B.Cu") (capping no) (covering (front no) (back no))
  (plugging (front no) (back no)) (filling no) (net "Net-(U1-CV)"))
 (segment (start 68.4609 49.205) (end 73.71 54.4541) (width 0.2) (layer "B.Cu") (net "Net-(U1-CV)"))
 (segment (start 68.025 49.205) (end 68.4609 49.205) (width 0.2) (layer "B.Cu") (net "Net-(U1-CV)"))
 (segment (start 77.606 50.9327) (end 77.606 42.406) (width 0.2) (layer "F.Cu") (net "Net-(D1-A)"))
 (segment (start 74.4777 52.1102) (end 76.4285 52.1102) (width 0.2) (layer "F.Cu") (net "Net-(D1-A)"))
 (segment (start 73.76 51.3925) (end 74.4777 52.1102) (width 0.2) (layer "F.Cu") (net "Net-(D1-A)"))
 (segment (start 76.4285 52.1102) (end 77.606 50.9327) (width 0.2) (layer "F.Cu") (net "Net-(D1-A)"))
 (segment (start 77.606 42.406) (end 75.8 40.6) (width 0.2) (layer "F.Cu") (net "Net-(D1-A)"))
 (segment (start 74.686 49.8055) (end 73.9792 50.5123) (width 0.2) (layer "F.Cu") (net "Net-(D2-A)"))
 (segment (start 76.8026 47.2103) (end 76.8026 48.2187) (width 0.2) (layer "F.Cu") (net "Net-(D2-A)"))
 (segment (start 73.9792 50.5123) (end 72.7277 50.5123) (width 0.2) (layer "F.Cu") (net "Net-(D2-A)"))
 (segment (start 74.686 49.209) (end 74.686 49.8055) (width 0.2) (layer "F.Cu") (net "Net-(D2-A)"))
 (segment (start 75.1007 46.7651) (end 76.3574 46.7651) (width 0.2) (layer "F.Cu") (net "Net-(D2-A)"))
 (segment (start 75.8 44.1) (end 74.7696 45.1304) (width 0.2) (layer "F.Cu") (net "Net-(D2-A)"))
 (segment (start 76.8026 48.2187) (end 76.4638 48.5575) (width 0.2) (layer "F.Cu") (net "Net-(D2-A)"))
 (segment (start 74.7696 45.1304) (end 74.7696 46.434) (width 0.2) (layer "F.Cu") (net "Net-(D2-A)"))
 (segment (start 76.3574 46.7651) (end 76.8026 47.2103) (width 0.2) (layer "F.Cu") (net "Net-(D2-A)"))
 (segment (start 76.4638 48.5575) (end 75.3375 48.5575) (width 0.2) (layer "F.Cu") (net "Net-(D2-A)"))
 (segment (start 74.7696 46.434) (end 75.1007 46.7651) (width 0.2) (layer "F.Cu") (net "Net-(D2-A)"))
 (segment (start 75.3375 48.5575) (end 74.686 49.209) (width 0.2) (layer "F.Cu") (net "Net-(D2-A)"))
 (segment (start 72.7277 50.5123) (end 71.86 51.38) (width 0.2) (layer "F.Cu") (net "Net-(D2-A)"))
 (segment (start 75.8 47.7) (end 75.5132 47.7) (width 0.2) (layer "F.Cu") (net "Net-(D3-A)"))
 (segment (start 71.9436 49.21) (end 69.9 51.2536) (width 0.2) (layer "F.Cu") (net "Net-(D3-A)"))
 (segment (start 69.9 51.2536) (end 69.9 51.3875) (width 0.2) (layer "F.Cu") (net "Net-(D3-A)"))
 (segment (start 74.0032 49.21) (end 71.9436 49.21) (width 0.2) (layer "F.Cu") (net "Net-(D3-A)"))
 (segment (start 75.5132 47.7) (end 74.0032 49.21) (width 0.2) (layer "F.Cu") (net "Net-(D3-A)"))
 (segment (start 71.4454 47.2061) (end 71.9815 46.67) (width 0.2) (layer "F.Cu") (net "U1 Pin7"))
 (segment (start 67.96 51.3675) (end 68.2225 51.3675) (width 0.2) (layer "F.Cu") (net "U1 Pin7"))
 (segment (start 68.2225 51.3675) (end 71.4454 48.1446) (width 0.2) (layer "F.Cu") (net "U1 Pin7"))
 (segment (start 71.4454 48.1446) (end 71.4454 47.2061) (width 0.2) (layer "F.Cu") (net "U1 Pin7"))
 (segment (start 71.9815 46.67) (end 73.9671 46.67) (width 0.2) (layer "F.Cu") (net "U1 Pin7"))
 (segment (start 74.34 46.2971) (end 74.34 36.9) (width 0.2) (layer "F.Cu") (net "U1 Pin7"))
 (segment (start 73.9671 46.67) (end 74.34 46.2971) (width 0.2) (layer "F.Cu") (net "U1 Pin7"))
 (segment (start 66.6704 38.0352) (end 66.6704 42.2357) (width 0.2) (layer "B.Cu") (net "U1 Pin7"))
 (segment (start 69.3431 45.7449) (end 68.423 46.665) (width 0.2) (layer "B.Cu") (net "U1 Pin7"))
 (segment (start 74.34 36.9) (end 73.2792 35.8392) (width 0.2) (layer "B.Cu") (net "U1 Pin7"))
 (segment (start 68.8664 35.8392) (end 66.6704 38.0352) (width 0.2) (layer "B.Cu") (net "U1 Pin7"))
 (segment (start 66.6704 42.2357) (end 69.3431 44.9084) (width 0.2) (layer "B.Cu") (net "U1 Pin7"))
 (segment (start 68.423 46.665) (end 68.025 46.665) (width 0.2) (layer "B.Cu") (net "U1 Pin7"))
 (segment (start 69.3431 44.9084) (end 69.3431 45.7449) (width 0.2) (layer "B.Cu") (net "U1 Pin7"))
 (segment (start 73.2792 35.8392) (end 68.8664 35.8392) (width 0.2) (layer "B.Cu") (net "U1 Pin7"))
 (segment (start 67.96 53.1925) (end 66.3293 51.5618) (width 0.2) (layer "F.Cu") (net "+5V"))
 (segment (start 66.3293 51.5618) (end 66.3293 49.3871) (width 0.2) (layer "F.Cu") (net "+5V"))
 (segment (start 72.975 39.877) (end 72.975 40.955) (width 0.2) (layer "F.Cu") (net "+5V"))
 (segment (start 73.5254 39.3266) (end 72.975 39.877) (width 0.2) (layer "F.Cu") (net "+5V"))
 (via (at 66.3293 49.3871) (size 0.6) (drill 0.3) (layers "F.Cu" "B.Cu") (capping no) (covering (front no) (back no))
  (plugging (front no) (back no)) (filling no) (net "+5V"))
 (via (at 73.5254 39.3266) (size 0.6) (drill 0.3) (layers "F.Cu" "B.Cu") (capping no) (covering (front no) (back no))
  (plugging (front no) (back no)) (filling no) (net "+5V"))
 (segment (start 77.5068 42.716) (end 74.1174 39.3266) (width 0.2) (layer "B.Cu") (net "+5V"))
 (segment (start 74.1174 39.3266) (end 73.5254 39.3266) (width 0.2) (layer "B.Cu") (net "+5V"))
 (segment (start 77.5068 45.0735) (end 77.5068 42.716) (width 0.2) (layer "B.Cu") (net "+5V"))
 (segment (start 67.6287 45.395) (end 66.7241 46.2996) (width 0.2) (layer "B.Cu") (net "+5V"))
 (segment (start 66.7241 48.2519) (end 67.0422 48.57) (width 0.2) (layer "B.Cu") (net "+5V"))
 (segment (start 66.3293 49.2829) (end 66.3293 49.3871) (width 0.2) (layer "B.Cu") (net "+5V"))
 (segment (start 72.34 48.57) (end 72.975 49.205) (width 0.2) (layer "B.Cu") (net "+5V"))
 (segment (start 68.025 45.395) (end 67.6287 45.395) (width 0.2) (layer "B.Cu") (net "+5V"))
 (segment (start 72.975 49.205) (end 73.3753 49.205) (width 0.2) (layer "B.Cu") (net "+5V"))
 (segment (start 67.0422 48.57) (end 72.34 48.57) (width 0.2) (layer "B.Cu") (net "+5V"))
 (segment (start 66.7241 46.2996) (end 66.7241 48.2519) (width 0.2) (layer "B.Cu") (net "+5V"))
 (segment (start 67.0422 48.57) (end 66.3293 49.2829) (width 0.2) (layer "B.Cu") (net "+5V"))
 (segment (start 73.3753 49.205) (end 77.5068 45.0735) (width 0.2) (layer "B.Cu") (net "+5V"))
 (segment (start 67.2888 54.0318) (end 65.694 52.437) (width 0.2) (layer "F.Cu") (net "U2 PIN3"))
 (segment (start 65.694 52.437) (end 65.694 45.4189) (width 0.2) (layer "F.Cu") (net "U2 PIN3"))
 (segment (start 65.694 45.4189) (end 67.6179 43.495) (width 0.2) (layer "F.Cu") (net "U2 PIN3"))
 (segment (start 67.6179 43.495) (end 68.025 43.495) (width 0.2) (layer "F.Cu") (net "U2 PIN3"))
 (segment (start 69.9 53.2125) (end 69.0807 54.0318) (width 0.2) (layer "F.Cu") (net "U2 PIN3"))
 (segment (start 69.0807 54.0318) (end 67.2888 54.0318) (width 0.2) (layer "F.Cu") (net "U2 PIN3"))
 (segment (start 65.2923 44.613) (end 65.2923 52.6052) (width 0.2) (layer "F.Cu") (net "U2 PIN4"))
 (segment (start 69.3023 43.8324) (end 69.3023 43.1576) (width 0.2) (layer "F.Cu") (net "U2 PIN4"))
 (segment (start 68.025 44.765) (end 68.3697 44.765) (width 0.2) (layer "F.Cu") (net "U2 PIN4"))
 (segment (start 69.0374 42.8927) (end 67.0126 42.8927) (width 0.2) (layer "F.Cu") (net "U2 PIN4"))
 (segment (start 69.3023 43.1576) (end 69.0374 42.8927) (width 0.2) (layer "F.Cu") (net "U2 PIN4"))
 (segment (start 65.2923 52.6052) (end 67.1624 54.4753) (width 0.2) (layer "F.Cu") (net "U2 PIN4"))
 (segment (start 68.3697 44.765) (end 69.3023 43.8324) (width 0.2) (layer "F.Cu") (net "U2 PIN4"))
 (segment (start 67.1624 54.4753) (end 70.5897 54.4753) (width 0.2) (layer "F.Cu") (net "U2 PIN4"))
 (segment (start 67.0126 42.8927) (end 65.2923 44.613) (width 0.2) (layer "F.Cu") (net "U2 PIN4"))
 (segment (start 70.5897 54.4753) (end 71.86 53.205) (width 0.2) (layer "F.Cu") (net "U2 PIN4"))
 (segment (start 73.76 53.2175) (end 74.53 53.9875) (width 0.2) (layer "F.Cu") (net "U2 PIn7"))
 (segment (start 74.53 53.9875) (end 74.53 54.2275) (width 0.2) (layer "F.Cu") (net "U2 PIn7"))
 (segment (start 68.8881 48.575) (end 69.5251 49.212) (width 0.2) (layer "F.Cu") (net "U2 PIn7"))
 (segment (start 68.025 48.575) (end 68.8881 48.575) (width 0.2) (layer "F.Cu") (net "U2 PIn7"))
 (via (at 69.5251 49.212) (size 0.6) (drill 0.3) (layers "F.Cu" "B.Cu") (capping no) (covering (front no) (back no))
  (plugging (front no) (back no)) (filling no) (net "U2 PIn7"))
 (via (at 74.53 54.2275) (size 0.6) (drill 0.3) (layers "F.Cu" "B.Cu") (capping no) (covering (front no) (back no))
  (plugging (front no) (back no)) (filling no) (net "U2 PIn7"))
 (segment (start 69.5251 49.2226) (end 74.53 54.2275) (width 0.2) (layer "B.Cu") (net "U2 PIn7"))
 (segment (start 69.5251 49.212) (end 69.5251 49.2226) (width 0.2) (layer "B.Cu") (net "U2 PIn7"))
 (segment (start 71.1908 45.33) (end 71.6975 44.8233) (width 0.2) (layer "F.Cu") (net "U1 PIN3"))
 (segment (start 71.6975 44.8233) (end 71.6975 44.4268) (width 0.2) (layer "F.Cu") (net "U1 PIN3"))
 (segment (start 72.6293 43.495) (end 72.975 43.495) (width 0.2) (layer "F.Cu") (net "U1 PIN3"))
 (segment (start 71.6975 44.4268) (end 72.6293 43.495) (width 0.2) (layer "F.Cu") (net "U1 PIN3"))
 (via (at 71.1908 45.33) (size 0.6) (drill 0.3) (layers "F.Cu" "B.Cu") (capping no) (covering (front no) (back no))
  (plugging (front no) (back no)) (filling no) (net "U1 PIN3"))
 (segment (start 74.2795 46.9872) (end 74.2795 46.3212) (width 0.2) (layer "B.Cu") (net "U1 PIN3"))
 (segment (start 73.3317 47.935) (end 74.2795 46.9872) (width 0.2) (layer "B.Cu") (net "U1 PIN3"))
 (segment (start 73.9883 46.03) (end 71.8908 46.03) (width 0.2) (layer "B.Cu") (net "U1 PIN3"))
 (segment (start 74.2795 46.3212) (end 73.9883 46.03) (width 0.2) (layer "B.Cu") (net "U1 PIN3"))
 (segment (start 72.975 47.935) (end 73.3317 47.935) (width 0.2) (layer "B.Cu") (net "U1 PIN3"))
 (segment (start 71.8908 46.03) (end 71.1908 45.33) (width 0.2) (layer "B.Cu") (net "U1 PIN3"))
 (segment (start 72.3078 41.5578) (end 68.6278 41.5578) (width 0.2) (layer "F.Cu") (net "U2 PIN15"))
 (segment (start 68.6278 41.5578) (end 68.025 40.955) (width 0.2) (layer "F.Cu") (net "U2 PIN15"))
 (segment (start 72.975 42.225) (end 72.3078 41.5578) (width 0.2) (layer "F.Cu") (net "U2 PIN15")))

